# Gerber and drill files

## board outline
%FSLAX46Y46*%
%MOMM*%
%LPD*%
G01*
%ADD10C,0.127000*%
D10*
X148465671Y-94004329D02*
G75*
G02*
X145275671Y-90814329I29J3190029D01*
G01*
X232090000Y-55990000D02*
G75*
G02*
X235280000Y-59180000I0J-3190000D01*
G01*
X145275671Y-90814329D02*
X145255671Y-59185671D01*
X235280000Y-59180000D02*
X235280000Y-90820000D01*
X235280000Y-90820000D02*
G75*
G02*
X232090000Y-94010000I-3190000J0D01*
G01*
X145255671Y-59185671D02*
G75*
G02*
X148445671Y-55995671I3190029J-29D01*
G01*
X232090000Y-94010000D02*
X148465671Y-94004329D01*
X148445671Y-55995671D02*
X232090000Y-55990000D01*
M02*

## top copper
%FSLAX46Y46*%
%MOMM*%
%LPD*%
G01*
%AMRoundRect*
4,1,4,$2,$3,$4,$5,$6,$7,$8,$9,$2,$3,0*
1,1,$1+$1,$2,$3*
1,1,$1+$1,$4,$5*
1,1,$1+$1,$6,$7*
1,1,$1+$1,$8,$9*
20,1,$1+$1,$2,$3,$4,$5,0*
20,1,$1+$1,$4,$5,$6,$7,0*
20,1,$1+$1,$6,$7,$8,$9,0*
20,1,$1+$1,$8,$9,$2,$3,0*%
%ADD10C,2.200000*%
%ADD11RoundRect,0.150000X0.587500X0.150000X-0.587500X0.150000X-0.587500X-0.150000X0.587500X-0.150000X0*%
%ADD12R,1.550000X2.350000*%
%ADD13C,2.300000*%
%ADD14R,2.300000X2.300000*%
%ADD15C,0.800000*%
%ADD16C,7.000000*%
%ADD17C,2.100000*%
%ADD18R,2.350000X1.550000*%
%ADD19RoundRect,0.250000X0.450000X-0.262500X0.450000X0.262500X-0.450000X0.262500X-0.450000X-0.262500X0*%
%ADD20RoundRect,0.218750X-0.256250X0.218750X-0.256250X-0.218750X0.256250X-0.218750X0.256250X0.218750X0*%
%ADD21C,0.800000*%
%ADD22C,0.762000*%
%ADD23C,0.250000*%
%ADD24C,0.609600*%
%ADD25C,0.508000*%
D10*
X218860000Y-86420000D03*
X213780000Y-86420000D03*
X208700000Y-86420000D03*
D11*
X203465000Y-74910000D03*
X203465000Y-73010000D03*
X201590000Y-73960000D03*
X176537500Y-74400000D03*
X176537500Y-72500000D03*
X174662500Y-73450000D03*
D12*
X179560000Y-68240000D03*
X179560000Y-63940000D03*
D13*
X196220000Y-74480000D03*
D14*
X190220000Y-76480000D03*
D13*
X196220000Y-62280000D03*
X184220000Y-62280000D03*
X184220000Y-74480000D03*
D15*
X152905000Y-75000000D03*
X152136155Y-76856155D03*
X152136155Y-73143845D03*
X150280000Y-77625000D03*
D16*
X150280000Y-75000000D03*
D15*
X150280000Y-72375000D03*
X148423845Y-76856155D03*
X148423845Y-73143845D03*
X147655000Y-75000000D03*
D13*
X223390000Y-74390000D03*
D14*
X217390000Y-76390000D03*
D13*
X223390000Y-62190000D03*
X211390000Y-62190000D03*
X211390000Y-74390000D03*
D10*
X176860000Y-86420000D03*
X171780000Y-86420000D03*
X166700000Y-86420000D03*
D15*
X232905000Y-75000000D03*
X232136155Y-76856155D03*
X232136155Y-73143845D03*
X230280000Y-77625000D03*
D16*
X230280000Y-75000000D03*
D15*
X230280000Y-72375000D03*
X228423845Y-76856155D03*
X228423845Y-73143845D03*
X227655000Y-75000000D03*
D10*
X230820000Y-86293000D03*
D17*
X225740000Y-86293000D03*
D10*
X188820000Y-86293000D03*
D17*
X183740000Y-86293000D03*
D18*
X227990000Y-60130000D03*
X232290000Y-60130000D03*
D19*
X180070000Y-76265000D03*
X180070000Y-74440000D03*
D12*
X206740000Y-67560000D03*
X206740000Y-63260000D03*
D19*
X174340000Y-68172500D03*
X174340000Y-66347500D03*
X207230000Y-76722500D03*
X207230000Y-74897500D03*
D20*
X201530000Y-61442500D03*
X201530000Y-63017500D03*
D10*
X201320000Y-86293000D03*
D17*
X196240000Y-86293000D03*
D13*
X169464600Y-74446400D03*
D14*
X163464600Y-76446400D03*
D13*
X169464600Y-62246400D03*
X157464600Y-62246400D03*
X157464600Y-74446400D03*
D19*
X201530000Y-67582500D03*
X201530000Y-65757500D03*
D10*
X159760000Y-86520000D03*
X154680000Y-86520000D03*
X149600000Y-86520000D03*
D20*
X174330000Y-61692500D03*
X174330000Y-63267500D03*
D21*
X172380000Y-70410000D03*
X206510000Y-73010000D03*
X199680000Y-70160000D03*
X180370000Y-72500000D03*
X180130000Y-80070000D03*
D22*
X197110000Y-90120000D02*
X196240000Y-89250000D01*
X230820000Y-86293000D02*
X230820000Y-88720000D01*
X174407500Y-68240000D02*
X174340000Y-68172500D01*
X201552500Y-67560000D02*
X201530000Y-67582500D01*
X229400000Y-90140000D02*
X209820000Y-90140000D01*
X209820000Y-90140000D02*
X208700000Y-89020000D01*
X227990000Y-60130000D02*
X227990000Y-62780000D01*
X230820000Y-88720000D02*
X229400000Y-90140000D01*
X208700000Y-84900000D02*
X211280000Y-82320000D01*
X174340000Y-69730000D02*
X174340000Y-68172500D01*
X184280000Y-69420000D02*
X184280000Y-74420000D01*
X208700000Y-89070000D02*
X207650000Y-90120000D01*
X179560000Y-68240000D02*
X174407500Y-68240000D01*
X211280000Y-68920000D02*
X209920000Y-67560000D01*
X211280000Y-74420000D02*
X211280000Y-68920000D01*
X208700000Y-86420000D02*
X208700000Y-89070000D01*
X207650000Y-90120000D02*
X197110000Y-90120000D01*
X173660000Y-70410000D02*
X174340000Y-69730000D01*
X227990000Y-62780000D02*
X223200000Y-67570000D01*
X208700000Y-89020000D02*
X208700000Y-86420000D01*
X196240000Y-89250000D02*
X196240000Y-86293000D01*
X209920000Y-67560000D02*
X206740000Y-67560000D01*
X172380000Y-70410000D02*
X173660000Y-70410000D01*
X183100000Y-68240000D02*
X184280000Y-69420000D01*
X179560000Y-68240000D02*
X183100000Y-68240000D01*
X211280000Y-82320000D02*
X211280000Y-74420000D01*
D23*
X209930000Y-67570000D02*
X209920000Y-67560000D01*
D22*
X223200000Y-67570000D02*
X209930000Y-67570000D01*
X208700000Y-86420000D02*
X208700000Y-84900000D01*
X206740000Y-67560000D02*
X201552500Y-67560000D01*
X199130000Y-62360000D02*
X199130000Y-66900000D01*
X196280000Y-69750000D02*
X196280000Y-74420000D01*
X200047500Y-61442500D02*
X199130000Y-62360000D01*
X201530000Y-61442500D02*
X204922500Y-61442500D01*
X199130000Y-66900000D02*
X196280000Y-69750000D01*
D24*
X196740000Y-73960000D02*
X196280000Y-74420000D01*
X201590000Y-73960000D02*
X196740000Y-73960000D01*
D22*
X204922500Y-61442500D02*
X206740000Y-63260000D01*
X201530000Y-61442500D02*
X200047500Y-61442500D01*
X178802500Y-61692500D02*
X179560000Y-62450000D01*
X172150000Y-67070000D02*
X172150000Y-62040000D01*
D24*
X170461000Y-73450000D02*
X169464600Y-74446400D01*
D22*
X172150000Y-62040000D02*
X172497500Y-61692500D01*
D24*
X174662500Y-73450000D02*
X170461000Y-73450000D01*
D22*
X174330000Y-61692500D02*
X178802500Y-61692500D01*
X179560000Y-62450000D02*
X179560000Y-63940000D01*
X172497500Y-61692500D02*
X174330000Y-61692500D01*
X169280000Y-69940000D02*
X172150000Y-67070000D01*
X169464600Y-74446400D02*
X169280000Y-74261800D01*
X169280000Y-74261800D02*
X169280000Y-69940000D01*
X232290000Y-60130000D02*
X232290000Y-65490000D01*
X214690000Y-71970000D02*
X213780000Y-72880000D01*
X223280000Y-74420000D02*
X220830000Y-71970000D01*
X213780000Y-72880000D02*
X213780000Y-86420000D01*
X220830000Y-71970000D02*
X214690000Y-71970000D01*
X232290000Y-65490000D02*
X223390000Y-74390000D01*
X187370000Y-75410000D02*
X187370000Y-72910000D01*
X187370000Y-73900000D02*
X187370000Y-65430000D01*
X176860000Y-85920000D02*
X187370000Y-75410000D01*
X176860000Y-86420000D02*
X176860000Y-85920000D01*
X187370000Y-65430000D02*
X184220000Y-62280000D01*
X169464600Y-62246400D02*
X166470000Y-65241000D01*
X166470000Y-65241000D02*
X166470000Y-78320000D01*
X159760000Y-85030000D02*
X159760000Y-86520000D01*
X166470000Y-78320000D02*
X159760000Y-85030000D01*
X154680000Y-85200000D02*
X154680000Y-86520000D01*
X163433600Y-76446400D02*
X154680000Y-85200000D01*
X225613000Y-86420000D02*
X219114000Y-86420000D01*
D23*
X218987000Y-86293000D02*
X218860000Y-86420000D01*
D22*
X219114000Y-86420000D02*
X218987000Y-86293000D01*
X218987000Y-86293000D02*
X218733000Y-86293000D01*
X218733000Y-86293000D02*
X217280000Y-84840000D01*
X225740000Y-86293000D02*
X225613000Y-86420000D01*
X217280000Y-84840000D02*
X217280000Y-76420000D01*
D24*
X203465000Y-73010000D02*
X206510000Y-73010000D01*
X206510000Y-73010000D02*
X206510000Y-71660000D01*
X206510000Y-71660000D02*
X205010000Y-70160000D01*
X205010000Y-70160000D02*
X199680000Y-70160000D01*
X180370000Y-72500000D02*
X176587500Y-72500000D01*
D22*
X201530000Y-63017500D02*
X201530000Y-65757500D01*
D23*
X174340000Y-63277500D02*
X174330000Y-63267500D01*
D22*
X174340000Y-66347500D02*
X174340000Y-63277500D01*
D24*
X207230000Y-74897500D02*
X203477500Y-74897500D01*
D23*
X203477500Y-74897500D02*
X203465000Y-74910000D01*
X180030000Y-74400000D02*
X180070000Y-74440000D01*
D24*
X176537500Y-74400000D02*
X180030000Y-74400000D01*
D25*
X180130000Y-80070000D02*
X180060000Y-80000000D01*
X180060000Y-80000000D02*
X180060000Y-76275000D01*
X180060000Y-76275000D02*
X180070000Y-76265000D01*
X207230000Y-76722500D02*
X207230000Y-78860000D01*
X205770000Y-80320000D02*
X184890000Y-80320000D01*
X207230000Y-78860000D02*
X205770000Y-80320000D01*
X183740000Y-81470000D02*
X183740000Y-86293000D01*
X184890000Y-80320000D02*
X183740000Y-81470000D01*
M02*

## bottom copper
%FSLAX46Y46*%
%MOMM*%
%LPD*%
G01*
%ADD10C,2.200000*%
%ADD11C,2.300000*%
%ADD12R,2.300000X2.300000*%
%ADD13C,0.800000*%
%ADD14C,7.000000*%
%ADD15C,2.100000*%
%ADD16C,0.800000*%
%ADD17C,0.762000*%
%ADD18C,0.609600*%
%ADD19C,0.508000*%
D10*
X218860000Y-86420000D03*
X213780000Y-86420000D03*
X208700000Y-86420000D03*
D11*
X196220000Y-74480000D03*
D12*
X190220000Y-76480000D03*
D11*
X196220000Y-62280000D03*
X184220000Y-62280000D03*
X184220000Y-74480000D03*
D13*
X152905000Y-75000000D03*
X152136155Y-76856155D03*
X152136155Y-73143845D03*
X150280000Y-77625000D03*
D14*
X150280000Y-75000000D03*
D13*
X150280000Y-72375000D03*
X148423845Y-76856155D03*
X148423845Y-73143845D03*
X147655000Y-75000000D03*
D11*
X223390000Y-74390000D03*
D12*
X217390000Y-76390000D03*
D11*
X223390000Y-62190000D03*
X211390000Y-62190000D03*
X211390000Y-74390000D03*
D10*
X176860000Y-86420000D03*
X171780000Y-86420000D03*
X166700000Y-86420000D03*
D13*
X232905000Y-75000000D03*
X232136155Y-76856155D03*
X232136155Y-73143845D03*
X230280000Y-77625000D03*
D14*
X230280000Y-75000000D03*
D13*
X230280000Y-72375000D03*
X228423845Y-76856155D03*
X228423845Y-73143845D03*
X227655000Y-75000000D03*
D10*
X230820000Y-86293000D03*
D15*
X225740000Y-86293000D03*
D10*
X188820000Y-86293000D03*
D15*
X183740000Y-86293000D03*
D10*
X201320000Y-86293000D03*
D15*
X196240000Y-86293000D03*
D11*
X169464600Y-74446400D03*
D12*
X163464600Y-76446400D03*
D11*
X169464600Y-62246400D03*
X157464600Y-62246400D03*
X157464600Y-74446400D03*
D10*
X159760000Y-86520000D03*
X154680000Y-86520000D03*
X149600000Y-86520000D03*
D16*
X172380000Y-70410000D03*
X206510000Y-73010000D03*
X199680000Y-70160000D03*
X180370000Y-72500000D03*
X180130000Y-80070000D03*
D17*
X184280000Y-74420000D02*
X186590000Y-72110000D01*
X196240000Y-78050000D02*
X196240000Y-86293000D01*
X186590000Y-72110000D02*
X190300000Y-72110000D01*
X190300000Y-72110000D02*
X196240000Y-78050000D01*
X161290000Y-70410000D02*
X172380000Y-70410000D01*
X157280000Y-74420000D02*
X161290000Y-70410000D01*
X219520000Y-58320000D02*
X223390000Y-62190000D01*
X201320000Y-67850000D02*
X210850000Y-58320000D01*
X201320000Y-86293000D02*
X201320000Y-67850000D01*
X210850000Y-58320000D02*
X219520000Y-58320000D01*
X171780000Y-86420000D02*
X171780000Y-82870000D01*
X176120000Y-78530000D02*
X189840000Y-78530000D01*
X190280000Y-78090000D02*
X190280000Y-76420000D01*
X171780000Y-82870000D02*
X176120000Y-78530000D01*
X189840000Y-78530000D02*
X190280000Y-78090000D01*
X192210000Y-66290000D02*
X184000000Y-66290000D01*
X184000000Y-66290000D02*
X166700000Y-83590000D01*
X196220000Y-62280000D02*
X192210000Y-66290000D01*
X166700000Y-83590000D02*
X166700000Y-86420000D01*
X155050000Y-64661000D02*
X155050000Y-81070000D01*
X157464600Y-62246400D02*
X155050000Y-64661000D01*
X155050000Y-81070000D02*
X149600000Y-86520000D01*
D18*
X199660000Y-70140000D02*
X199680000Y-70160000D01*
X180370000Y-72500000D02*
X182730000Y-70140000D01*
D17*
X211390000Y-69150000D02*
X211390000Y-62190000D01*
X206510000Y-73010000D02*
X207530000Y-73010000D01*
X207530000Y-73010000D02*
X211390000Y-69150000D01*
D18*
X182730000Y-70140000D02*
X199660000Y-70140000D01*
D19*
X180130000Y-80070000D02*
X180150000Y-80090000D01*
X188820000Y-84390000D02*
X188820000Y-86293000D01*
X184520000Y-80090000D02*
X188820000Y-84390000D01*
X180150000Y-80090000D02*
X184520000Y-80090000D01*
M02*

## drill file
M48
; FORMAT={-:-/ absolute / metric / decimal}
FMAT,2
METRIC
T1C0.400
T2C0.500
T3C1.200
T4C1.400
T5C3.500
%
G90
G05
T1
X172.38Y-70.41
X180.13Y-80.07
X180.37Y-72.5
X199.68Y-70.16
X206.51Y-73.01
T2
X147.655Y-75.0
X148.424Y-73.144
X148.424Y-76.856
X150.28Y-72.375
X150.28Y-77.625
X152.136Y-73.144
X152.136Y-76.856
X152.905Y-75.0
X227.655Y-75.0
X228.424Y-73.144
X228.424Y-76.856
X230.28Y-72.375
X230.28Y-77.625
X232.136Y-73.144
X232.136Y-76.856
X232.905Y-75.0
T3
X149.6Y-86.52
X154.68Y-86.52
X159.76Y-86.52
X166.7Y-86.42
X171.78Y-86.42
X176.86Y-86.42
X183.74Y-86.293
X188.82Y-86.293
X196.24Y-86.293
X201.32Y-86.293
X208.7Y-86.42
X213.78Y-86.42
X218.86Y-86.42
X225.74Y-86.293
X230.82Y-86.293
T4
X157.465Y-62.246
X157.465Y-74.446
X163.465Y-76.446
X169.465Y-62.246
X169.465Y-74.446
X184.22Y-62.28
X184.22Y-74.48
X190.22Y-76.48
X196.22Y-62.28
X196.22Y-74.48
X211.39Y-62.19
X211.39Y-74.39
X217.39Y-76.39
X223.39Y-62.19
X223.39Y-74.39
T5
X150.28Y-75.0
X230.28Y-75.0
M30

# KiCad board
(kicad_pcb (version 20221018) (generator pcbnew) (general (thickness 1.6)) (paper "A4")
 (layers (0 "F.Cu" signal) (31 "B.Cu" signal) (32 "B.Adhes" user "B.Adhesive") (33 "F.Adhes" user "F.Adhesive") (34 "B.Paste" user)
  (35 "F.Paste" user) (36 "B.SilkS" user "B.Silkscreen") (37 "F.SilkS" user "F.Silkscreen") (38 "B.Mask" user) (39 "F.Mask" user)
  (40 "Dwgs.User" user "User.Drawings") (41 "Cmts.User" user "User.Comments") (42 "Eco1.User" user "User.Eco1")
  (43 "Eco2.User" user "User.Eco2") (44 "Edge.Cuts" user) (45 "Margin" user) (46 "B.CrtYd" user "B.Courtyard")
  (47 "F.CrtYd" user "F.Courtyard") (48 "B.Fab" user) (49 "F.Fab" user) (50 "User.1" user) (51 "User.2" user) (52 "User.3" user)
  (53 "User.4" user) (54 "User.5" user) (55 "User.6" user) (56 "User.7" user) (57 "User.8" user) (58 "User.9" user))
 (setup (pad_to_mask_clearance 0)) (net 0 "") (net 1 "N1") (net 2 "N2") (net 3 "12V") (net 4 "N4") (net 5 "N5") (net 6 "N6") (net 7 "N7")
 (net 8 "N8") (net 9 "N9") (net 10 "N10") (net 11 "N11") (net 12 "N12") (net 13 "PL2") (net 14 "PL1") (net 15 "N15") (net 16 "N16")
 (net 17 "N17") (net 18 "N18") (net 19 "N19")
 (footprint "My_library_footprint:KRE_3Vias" (layer "F.Cu") (at 213.78 86.42 180)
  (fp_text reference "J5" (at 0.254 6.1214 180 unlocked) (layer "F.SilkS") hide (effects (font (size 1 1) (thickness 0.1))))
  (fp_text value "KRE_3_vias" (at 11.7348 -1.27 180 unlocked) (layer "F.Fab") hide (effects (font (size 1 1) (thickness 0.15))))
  (pad "1" thru_hole circle (at -5.08 0 180) (size 2.2 2.2) (drill 1.2) (layers "*.Cu" "*.Mask") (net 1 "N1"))
  (pad "2" thru_hole circle (at 0 0 180) (size 2.2 2.2) (drill 1.2) (layers "*.Cu" "*.Mask") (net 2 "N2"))
  (pad "3" thru_hole circle (at 5.08 0 180) (size 2.2 2.2) (drill 1.2) (layers "*.Cu" "*.Mask") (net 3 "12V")))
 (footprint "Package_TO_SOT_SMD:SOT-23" (layer "F.Cu") (at 202.5275 73.96 180)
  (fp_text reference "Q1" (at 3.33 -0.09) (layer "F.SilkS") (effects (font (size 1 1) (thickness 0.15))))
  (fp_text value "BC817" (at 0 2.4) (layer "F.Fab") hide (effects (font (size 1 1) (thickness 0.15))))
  (pad "1" smd roundrect (at -0.9375 -0.95 180) (size 1.475 0.6) (layers "F.Cu" "F.Paste" "F.Mask") (roundrect_rratio 0.25) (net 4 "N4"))
  (pad "2" smd roundrect (at -0.9375 0.95 180) (size 1.475 0.6) (layers "F.Cu" "F.Paste" "F.Mask") (roundrect_rratio 0.25) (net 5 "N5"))
  (pad "3" smd roundrect (at 0.9375 0 180) (size 1.475 0.6) (layers "F.Cu" "F.Paste" "F.Mask") (roundrect_rratio 0.25) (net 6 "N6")))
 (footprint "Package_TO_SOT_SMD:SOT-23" (layer "F.Cu") (at 175.6 73.45 180)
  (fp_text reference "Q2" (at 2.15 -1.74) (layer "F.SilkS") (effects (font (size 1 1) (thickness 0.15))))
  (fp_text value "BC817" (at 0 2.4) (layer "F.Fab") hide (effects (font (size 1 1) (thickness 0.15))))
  (pad "1" smd roundrect (at -0.9375 -0.95 180) (size 1.475 0.6) (layers "F.Cu" "F.Paste" "F.Mask") (roundrect_rratio 0.25) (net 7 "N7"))
  (pad "2" smd roundrect (at -0.9375 0.95 180) (size 1.475 0.6) (layers "F.Cu" "F.Paste" "F.Mask") (roundrect_rratio 0.25) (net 5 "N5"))
  (pad "3" smd roundrect (at 0.9375 0 180) (size 1.475 0.6) (layers "F.Cu" "F.Paste" "F.Mask") (roundrect_rratio 0.25) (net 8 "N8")))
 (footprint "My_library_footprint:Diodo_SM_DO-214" (layer "F.Cu") (at 179.56 66.09 90)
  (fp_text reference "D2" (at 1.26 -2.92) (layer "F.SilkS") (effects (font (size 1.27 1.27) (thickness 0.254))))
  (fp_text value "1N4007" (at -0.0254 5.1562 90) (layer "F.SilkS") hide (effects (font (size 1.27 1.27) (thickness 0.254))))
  (pad "1" smd rect (at -2.15 0 180) (size 1.55 2.35) (layers "F.Cu" "F.Paste" "F.Mask") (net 3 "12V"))
  (pad "2" smd rect (at 2.15 0 180) (size 1.55 2.35) (layers "F.Cu" "F.Paste" "F.Mask") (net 8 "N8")))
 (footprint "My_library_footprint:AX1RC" (layer "F.Cu") (at 190.22 76.48 90)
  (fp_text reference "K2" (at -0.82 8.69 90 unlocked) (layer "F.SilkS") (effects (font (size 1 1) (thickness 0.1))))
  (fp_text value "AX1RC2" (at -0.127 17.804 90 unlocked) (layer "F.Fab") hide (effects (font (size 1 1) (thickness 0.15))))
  (pad "1" thru_hole circle (at 2 6 90) (size 2.3 2.3) (drill 1.4) (layers "*.Cu" "*.Mask") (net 6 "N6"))
  (pad "2" thru_hole rect (at 0 0 90) (size 2.3 2.3) (drill 1.4) (layers "*.Cu" "*.Mask") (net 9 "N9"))
  (pad "3" thru_hole circle (at 14.2 6 90) (size 2.3 2.3) (drill 1.4) (layers "*.Cu" "*.Mask") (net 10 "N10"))
  (pad "4" thru_hole circle (at 14.2 -6 90) (size 2.3 2.3) (drill 1.4) (layers "*.Cu" "*.Mask") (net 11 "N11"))
  (pad "5" thru_hole circle (at 2 -6 90) (size 2.3 2.3) (drill 1.4) (layers "*.Cu" "*.Mask") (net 3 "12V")))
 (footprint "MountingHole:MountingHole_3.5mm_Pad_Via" (layer "F.Cu") (at 150.28 75 180)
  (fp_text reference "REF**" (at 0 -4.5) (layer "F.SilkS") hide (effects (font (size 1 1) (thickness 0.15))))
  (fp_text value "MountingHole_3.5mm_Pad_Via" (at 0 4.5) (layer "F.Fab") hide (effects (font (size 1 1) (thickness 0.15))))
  (pad "1" thru_hole circle (at -2.625 0 180) (size 0.8 0.8) (drill 0.5) (layers "*.Cu" "*.Mask"))
  (pad "1" thru_hole circle (at -1.856155 -1.856155 180) (size 0.8 0.8) (drill 0.5) (layers "*.Cu" "*.Mask"))
  (pad "1" thru_hole circle (at -1.856155 1.856155 180) (size 0.8 0.8) (drill 0.5) (layers "*.Cu" "*.Mask"))
  (pad "1" thru_hole circle (at 0 -2.625 180) (size 0.8 0.8) (drill 0.5) (layers "*.Cu" "*.Mask"))
  (pad "1" thru_hole circle (at 0 0 180) (size 7 7) (drill 3.5) (layers "*.Cu" "*.Mask"))
  (pad "1" thru_hole circle (at 0 2.625 180) (size 0.8 0.8) (drill 0.5) (layers "*.Cu" "*.Mask"))
  (pad "1" thru_hole circle (at 1.856155 -1.856155 180) (size 0.8 0.8) (drill 0.5) (layers "*.Cu" "*.Mask"))
  (pad "1" thru_hole circle (at 1.856155 1.856155 180) (size 0.8 0.8) (drill 0.5) (layers "*.Cu" "*.Mask"))
  (pad "1" thru_hole circle (at 2.625 0 180) (size 0.8 0.8) (drill 0.5) (layers "*.Cu" "*.Mask")))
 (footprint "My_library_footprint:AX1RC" (layer "F.Cu") (at 217.39 76.39 90)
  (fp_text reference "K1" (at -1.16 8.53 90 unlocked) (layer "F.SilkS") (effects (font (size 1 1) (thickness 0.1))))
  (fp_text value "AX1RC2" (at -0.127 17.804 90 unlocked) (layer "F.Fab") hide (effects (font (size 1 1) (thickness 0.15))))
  (pad "1" thru_hole circle (at 2 6 90) (size 2.3 2.3) (drill 1.4) (layers "*.Cu" "*.Mask") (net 2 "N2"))
  (pad "2" thru_hole rect (at 0 0 90) (size 2.3 2.3) (drill 1.4) (layers "*.Cu" "*.Mask") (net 1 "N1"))
  (pad "3" thru_hole circle (at 14.2 6 90) (size 2.3 2.3) (drill 1.4) (layers "*.Cu" "*.Mask") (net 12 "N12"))
  (pad "4" thru_hole circle (at 14.2 -6 90) (size 2.3 2.3) (drill 1.4) (layers "*.Cu" "*.Mask") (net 5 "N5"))
  (pad "5" thru_hole circle (at 2 -6 90) (size 2.3 2.3) (drill 1.4) (layers "*.Cu" "*.Mask") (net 3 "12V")))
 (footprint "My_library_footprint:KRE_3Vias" (layer "F.Cu") (at 171.78 86.42 180)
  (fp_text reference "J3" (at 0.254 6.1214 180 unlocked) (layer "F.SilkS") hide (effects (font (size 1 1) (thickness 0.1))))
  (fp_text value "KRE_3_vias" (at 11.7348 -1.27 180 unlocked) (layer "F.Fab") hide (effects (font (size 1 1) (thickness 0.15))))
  (pad "1" thru_hole circle (at -5.08 0 180) (size 2.2 2.2) (drill 1.2) (layers "*.Cu" "*.Mask") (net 11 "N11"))
  (pad "2" thru_hole circle (at 0 0 180) (size 2.2 2.2) (drill 1.2) (layers "*.Cu" "*.Mask") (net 9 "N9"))
  (pad "3" thru_hole circle (at 5.08 0 180) (size 2.2 2.2) (drill 1.2) (layers "*.Cu" "*.Mask") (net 10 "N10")))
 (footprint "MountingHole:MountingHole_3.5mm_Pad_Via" (layer "F.Cu") (at 230.28 75 180)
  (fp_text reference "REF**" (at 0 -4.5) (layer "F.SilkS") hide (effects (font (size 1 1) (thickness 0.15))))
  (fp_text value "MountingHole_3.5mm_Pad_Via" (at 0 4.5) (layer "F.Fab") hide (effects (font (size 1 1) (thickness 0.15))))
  (pad "1" thru_hole circle (at -2.625 0 180) (size 0.8 0.8) (drill 0.5) (layers "*.Cu" "*.Mask"))
  (pad "1" thru_hole circle (at -1.856155 -1.856155 180) (size 0.8 0.8) (drill 0.5) (layers "*.Cu" "*.Mask"))
  (pad "1" thru_hole circle (at -1.856155 1.856155 180) (size 0.8 0.8) (drill 0.5) (layers "*.Cu" "*.Mask"))
  (pad "1" thru_hole circle (at 0 -2.625 180) (size 0.8 0.8) (drill 0.5) (layers "*.Cu" "*.Mask"))
  (pad "1" thru_hole circle (at 0 0 180) (size 7 7) (drill 3.5) (layers "*.Cu" "*.Mask"))
  (pad "1" thru_hole circle (at 0 2.625 180) (size 0.8 0.8) (drill 0.5) (layers "*.Cu" "*.Mask"))
  (pad "1" thru_hole circle (at 1.856155 -1.856155 180) (size 0.8 0.8) (drill 0.5) (layers "*.Cu" "*.Mask"))
  (pad "1" thru_hole circle (at 1.856155 1.856155 180) (size 0.8 0.8) (drill 0.5) (layers "*.Cu" "*.Mask"))
  (pad "1" thru_hole circle (at 2.625 0 180) (size 0.8 0.8) (drill 0.5) (layers "*.Cu" "*.Mask")))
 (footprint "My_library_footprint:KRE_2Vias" (layer "F.Cu") (at 228.28 86.42 180)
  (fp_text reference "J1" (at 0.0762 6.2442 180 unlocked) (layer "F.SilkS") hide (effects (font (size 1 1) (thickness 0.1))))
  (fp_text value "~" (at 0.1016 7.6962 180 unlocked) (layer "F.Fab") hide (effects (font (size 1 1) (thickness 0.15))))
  (pad "1" thru_hole circle (at -2.54 0.127 180) (size 2.2 2.2) (drill 1.2) (layers "*.Cu" "*.Mask") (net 3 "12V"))
  (pad "2" thru_hole circle (at 2.54 0.127 180) (size 2.1 2.1) (drill 1.2) (layers "*.Cu" "*.Mask") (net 1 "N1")))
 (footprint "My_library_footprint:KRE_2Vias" (layer "F.Cu") (at 186.28 86.42 180)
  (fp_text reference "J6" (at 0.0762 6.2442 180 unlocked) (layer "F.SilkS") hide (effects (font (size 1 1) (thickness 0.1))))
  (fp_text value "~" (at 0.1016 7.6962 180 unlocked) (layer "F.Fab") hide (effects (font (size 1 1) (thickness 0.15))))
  (pad "1" thru_hole circle (at -2.54 0.127 180) (size 2.2 2.2) (drill 1.2) (layers "*.Cu" "*.Mask") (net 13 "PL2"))
  (pad "2" thru_hole circle (at 2.54 0.127 180) (size 2.1 2.1) (drill 1.2) (layers "*.Cu" "*.Mask") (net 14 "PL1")))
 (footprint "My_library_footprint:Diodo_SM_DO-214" (layer "F.Cu") (at 230.14 60.13)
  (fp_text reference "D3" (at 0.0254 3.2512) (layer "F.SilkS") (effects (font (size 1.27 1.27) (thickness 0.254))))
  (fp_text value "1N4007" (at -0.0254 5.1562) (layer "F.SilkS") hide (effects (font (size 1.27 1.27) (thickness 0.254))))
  (pad "1" smd rect (at -2.15 0 90) (size 1.55 2.35) (layers "F.Cu" "F.Paste" "F.Mask") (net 3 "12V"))
  (pad "2" smd rect (at 2.15 0 90) (size 1.55 2.35) (layers "F.Cu" "F.Paste" "F.Mask") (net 2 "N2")))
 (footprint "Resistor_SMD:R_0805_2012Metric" (layer "F.Cu") (at 180.07 75.3525 90)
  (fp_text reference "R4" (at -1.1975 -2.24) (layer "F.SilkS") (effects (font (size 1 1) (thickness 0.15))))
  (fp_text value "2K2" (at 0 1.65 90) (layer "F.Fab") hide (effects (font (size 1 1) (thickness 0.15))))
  (pad "1" smd roundrect (at -0.9125 0 90) (size 1.025 1.4) (layers "F.Cu" "F.Paste" "F.Mask") (roundrect_rratio 0.243902439) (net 13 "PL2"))
  (pad "2" smd roundrect (at 0.9125 0 90) (size 1.025 1.4) (layers "F.Cu" "F.Paste" "F.Mask") (roundrect_rratio 0.243902439) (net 7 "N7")))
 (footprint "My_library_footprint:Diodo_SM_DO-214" (layer "F.Cu") (at 206.74 65.41 90)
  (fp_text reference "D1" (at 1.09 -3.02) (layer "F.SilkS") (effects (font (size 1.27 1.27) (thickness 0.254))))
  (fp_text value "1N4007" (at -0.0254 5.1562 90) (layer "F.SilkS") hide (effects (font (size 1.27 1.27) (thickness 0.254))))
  (pad "1" smd rect (at -2.15 0 180) (size 1.55 2.35) (layers "F.Cu" "F.Paste" "F.Mask") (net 3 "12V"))
  (pad "2" smd rect (at 2.15 0 180) (size 1.55 2.35) (layers "F.Cu" "F.Paste" "F.Mask") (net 6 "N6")))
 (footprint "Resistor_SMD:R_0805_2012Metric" (layer "F.Cu") (at 174.34 67.26 90)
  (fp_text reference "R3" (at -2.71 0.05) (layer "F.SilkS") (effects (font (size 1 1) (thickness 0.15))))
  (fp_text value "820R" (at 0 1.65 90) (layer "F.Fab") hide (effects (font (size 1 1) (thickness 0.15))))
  (pad "1" smd roundrect (at -0.9125 0 90) (size 1.025 1.4) (layers "F.Cu" "F.Paste" "F.Mask") (roundrect_rratio 0.243902439) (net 3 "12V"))
  (pad "2" smd roundrect (at 0.9125 0 90) (size 1.025 1.4) (layers "F.Cu" "F.Paste" "F.Mask") (roundrect_rratio 0.243902439) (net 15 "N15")))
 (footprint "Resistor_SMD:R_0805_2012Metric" (layer "F.Cu") (at 207.23 75.81 90)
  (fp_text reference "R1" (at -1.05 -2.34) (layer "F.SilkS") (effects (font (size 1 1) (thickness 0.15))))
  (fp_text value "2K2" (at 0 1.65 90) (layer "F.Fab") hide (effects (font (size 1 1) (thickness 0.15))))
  (pad "1" smd roundrect (at -0.9125 0 90) (size 1.025 1.4) (layers "F.Cu" "F.Paste" "F.Mask") (roundrect_rratio 0.243902439) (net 14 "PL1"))
  (pad "2" smd roundrect (at 0.9125 0 90) (size 1.025 1.4) (layers "F.Cu" "F.Paste" "F.Mask") (roundrect_rratio 0.243902439) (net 4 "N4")))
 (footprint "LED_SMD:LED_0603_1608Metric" (layer "F.Cu") (at 201.53 62.23 -90)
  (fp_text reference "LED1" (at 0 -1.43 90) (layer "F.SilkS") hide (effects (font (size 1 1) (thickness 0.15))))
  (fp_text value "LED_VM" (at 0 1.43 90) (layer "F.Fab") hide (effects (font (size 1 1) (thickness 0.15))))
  (pad "1" smd roundrect (at -0.7875 0 270) (size 0.875 0.95) (layers "F.Cu" "F.Paste" "F.Mask") (roundrect_rratio 0.25) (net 6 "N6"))
  (pad "2" smd roundrect (at 0.7875 0 270) (size 0.875 0.95) (layers "F.Cu" "F.Paste" "F.Mask") (roundrect_rratio 0.25) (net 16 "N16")))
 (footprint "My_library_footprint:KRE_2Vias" (layer "F.Cu") (at 198.78 86.42 180)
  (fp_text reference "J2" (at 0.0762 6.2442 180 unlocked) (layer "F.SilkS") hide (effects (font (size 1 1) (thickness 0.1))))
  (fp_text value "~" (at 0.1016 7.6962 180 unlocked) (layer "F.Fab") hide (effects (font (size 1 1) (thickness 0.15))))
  (pad "1" thru_hole circle (at -2.54 0.127 180) (size 2.2 2.2) (drill 1.2) (layers "*.Cu" "*.Mask") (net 12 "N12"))
  (pad "2" thru_hole circle (at 2.54 0.127 180) (size 2.1 2.1) (drill 1.2) (layers "*.Cu" "*.Mask") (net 3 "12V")))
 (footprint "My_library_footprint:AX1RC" (layer "F.Cu") (at 163.4646 76.4464 90)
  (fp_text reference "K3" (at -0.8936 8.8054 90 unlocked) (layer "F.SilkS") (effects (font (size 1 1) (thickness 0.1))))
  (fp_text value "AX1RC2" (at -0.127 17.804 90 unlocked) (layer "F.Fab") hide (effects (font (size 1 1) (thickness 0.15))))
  (pad "1" thru_hole circle (at 2 6 90) (size 2.3 2.3) (drill 1.4) (layers "*.Cu" "*.Mask") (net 8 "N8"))
  (pad "2" thru_hole rect (at 0 0 90) (size 2.3 2.3) (drill 1.4) (layers "*.Cu" "*.Mask") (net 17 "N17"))
  (pad "3" thru_hole circle (at 14.2 6 90) (size 2.3 2.3) (drill 1.4) (layers "*.Cu" "*.Mask") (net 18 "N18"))
  (pad "4" thru_hole circle (at 14.2 -6 90) (size 2.3 2.3) (drill 1.4) (layers "*.Cu" "*.Mask") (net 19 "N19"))
  (pad "5" thru_hole circle (at 2 -6 90) (size 2.3 2.3) (drill 1.4) (layers "*.Cu" "*.Mask") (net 3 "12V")))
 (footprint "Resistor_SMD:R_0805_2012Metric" (layer "F.Cu") (at 201.53 66.67 90)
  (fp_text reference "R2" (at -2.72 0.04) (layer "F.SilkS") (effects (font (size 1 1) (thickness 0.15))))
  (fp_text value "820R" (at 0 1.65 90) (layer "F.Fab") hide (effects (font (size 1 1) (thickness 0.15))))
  (pad "1" smd roundrect (at -0.9125 0 90) (size 1.025 1.4) (layers "F.Cu" "F.Paste" "F.Mask") (roundrect_rratio 0.243902439) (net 3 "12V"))
  (pad "2" smd roundrect (at 0.9125 0 90) (size 1.025 1.4) (layers "F.Cu" "F.Paste" "F.Mask") (roundrect_rratio 0.243902439) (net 16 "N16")))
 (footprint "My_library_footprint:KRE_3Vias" (layer "F.Cu") (at 154.68 86.52 180)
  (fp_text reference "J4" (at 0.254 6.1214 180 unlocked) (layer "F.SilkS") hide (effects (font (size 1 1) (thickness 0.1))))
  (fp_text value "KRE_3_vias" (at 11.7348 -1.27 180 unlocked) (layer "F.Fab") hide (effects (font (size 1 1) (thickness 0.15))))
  (pad "1" thru_hole circle (at -5.08 0 180) (size 2.2 2.2) (drill 1.2) (layers "*.Cu" "*.Mask") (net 18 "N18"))
  (pad "2" thru_hole circle (at 0 0 180) (size 2.2 2.2) (drill 1.2) (layers "*.Cu" "*.Mask") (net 17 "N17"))
  (pad "3" thru_hole circle (at 5.08 0 180) (size 2.2 2.2) (drill 1.2) (layers "*.Cu" "*.Mask") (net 19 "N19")))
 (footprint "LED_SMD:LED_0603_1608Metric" (layer "F.Cu") (at 174.33 62.48 -90)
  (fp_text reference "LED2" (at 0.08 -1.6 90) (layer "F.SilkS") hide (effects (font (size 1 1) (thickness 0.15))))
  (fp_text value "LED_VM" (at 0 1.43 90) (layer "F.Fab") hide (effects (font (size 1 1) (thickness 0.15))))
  (pad "1" smd roundrect (at -0.7875 0 270) (size 0.875 0.95) (layers "F.Cu" "F.Paste" "F.Mask") (roundrect_rratio 0.25) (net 8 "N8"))
  (pad "2" smd roundrect (at 0.7875 0 270) (size 0.875 0.95) (layers "F.Cu" "F.Paste" "F.Mask") (roundrect_rratio 0.25) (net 15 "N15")))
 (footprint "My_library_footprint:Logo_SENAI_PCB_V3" (layer "B.Cu") (at 225.837083 67.344083 180)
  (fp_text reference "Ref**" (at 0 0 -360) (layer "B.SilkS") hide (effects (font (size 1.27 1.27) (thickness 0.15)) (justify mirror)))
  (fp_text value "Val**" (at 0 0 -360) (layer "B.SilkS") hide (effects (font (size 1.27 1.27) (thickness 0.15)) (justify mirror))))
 (gr_arc (start 148.465671 94.004329) (mid 146.21 93.07) (end 145.275671 90.814329) (stroke (width 0.127) (type default))
  (layer "Edge.Cuts"))
 (gr_arc (start 232.09 55.99) (mid 234.345671 56.924329) (end 235.28 59.18) (stroke (width 0.127) (type default)) (layer "Edge.Cuts"))
 (gr_line (start 145.275671 90.814329) (end 145.255671 59.185671) (stroke (width 0.127) (type default)) (layer "Edge.Cuts"))
 (gr_line (start 235.28 59.18) (end 235.28 90.82) (stroke (width 0.127) (type default)) (layer "Edge.Cuts"))
 (gr_arc (start 235.28 90.82) (mid 234.345671 93.075671) (end 232.09 94.01) (stroke (width 0.127) (type default)) (layer "Edge.Cuts"))
 (gr_arc (start 145.255671 59.185671) (mid 146.19 56.93) (end 148.445671 55.995671) (stroke (width 0.127) (type default))
  (layer "Edge.Cuts"))
 (gr_line (start 232.09 94.01) (end 148.465671 94.004329) (stroke (width 0.127) (type default)) (layer "Edge.Cuts"))
 (gr_line (start 148.445671 55.995671) (end 232.09 55.99) (stroke (width 0.127) (type default)) (layer "Edge.Cuts"))
 (segment (start 197.11 90.12) (end 196.24 89.25) (width 0.762) (layer "F.Cu") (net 3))
 (segment (start 230.82 86.293) (end 230.82 88.72) (width 0.762) (layer "F.Cu") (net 3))
 (segment (start 174.4075 68.24) (end 174.34 68.1725) (width 0.762) (layer "F.Cu") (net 3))
 (segment (start 201.5525 67.56) (end 201.53 67.5825) (width 0.762) (layer "F.Cu") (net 3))
 (segment (start 229.4 90.14) (end 209.82 90.14) (width 0.762) (layer "F.Cu") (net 3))
 (segment (start 209.82 90.14) (end 208.7 89.02) (width 0.762) (layer "F.Cu") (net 3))
 (segment (start 227.99 60.13) (end 227.99 62.78) (width 0.762) (layer "F.Cu") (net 3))
 (segment (start 230.82 88.72) (end 229.4 90.14) (width 0.762) (layer "F.Cu") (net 3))
 (segment (start 208.7 84.9) (end 211.28 82.32) (width 0.762) (layer "F.Cu") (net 3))
 (segment (start 174.34 69.73) (end 174.34 68.1725) (width 0.762) (layer "F.Cu") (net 3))
 (segment (start 184.28 69.42) (end 184.28 74.42) (width 0.762) (layer "F.Cu") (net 3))
 (segment (start 208.7 89.07) (end 207.65 90.12) (width 0.762) (layer "F.Cu") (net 3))
 (segment (start 179.56 68.24) (end 174.4075 68.24) (width 0.762) (layer "F.Cu") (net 3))
 (segment (start 211.28 68.92) (end 209.92 67.56) (width 0.762) (layer "F.Cu") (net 3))
 (segment (start 211.28 74.42) (end 211.28 68.92) (width 0.762) (layer "F.Cu") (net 3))
 (segment (start 208.7 86.42) (end 208.7 89.07) (width 0.762) (layer "F.Cu") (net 3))
 (segment (start 207.65 90.12) (end 197.11 90.12) (width 0.762) (layer "F.Cu") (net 3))
 (segment (start 173.66 70.41) (end 174.34 69.73) (width 0.762) (layer "F.Cu") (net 3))
 (segment (start 227.99 62.78) (end 223.2 67.57) (width 0.762) (layer "F.Cu") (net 3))
 (segment (start 208.7 89.02) (end 208.7 86.42) (width 0.762) (layer "F.Cu") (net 3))
 (segment (start 196.24 89.25) (end 196.24 86.293) (width 0.762) (layer "F.Cu") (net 3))
 (segment (start 209.92 67.56) (end 206.74 67.56) (width 0.762) (layer "F.Cu") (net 3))
 (segment (start 172.38 70.41) (end 173.66 70.41) (width 0.762) (layer "F.Cu") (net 3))
 (segment (start 183.1 68.24) (end 184.28 69.42) (width 0.762) (layer "F.Cu") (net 3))
 (segment (start 179.56 68.24) (end 183.1 68.24) (width 0.762) (layer "F.Cu") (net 3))
 (segment (start 211.28 82.32) (end 211.28 74.42) (width 0.762) (layer "F.Cu") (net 3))
 (segment (start 209.93 67.57) (end 209.92 67.56) (width 0.25) (layer "F.Cu") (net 3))
 (segment (start 223.2 67.57) (end 209.93 67.57) (width 0.762) (layer "F.Cu") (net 3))
 (segment (start 208.7 86.42) (end 208.7 84.9) (width 0.762) (layer "F.Cu") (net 3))
 (segment (start 206.74 67.56) (end 201.5525 67.56) (width 0.762) (layer "F.Cu") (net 3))
 (via (at 172.38 70.41) (size 0.8) (drill 0.4) (layers "F.Cu" "B.Cu") (free) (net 3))
 (segment (start 184.28 74.42) (end 186.59 72.11) (width 0.762) (layer "B.Cu") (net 3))
 (segment (start 196.24 78.05) (end 196.24 86.293) (width 0.762) (layer "B.Cu") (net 3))
 (segment (start 186.59 72.11) (end 190.3 72.11) (width 0.762) (layer "B.Cu") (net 3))
 (segment (start 190.3 72.11) (end 196.24 78.05) (width 0.762) (layer "B.Cu") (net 3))
 (segment (start 161.29 70.41) (end 172.38 70.41) (width 0.762) (layer "B.Cu") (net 3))
 (segment (start 157.28 74.42) (end 161.29 70.41) (width 0.762) (layer "B.Cu") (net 3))
 (segment (start 199.13 62.36) (end 199.13 66.9) (width 0.762) (layer "F.Cu") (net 6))
 (segment (start 196.28 69.75) (end 196.28 74.42) (width 0.762) (layer "F.Cu") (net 6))
 (segment (start 200.0475 61.4425) (end 199.13 62.36) (width 0.762) (layer "F.Cu") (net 6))
 (segment (start 201.53 61.4425) (end 204.9225 61.4425) (width 0.762) (layer "F.Cu") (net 6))
 (segment (start 199.13 66.9) (end 196.28 69.75) (width 0.762) (layer "F.Cu") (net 6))
 (segment (start 196.74 73.96) (end 196.28 74.42) (width 0.6096) (layer "F.Cu") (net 6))
 (segment (start 201.59 73.96) (end 196.74 73.96) (width 0.6096) (layer "F.Cu") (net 6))
 (segment (start 204.9225 61.4425) (end 206.74 63.26) (width 0.762) (layer "F.Cu") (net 6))
 (segment (start 201.53 61.4425) (end 200.0475 61.4425) (width 0.762) (layer "F.Cu") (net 6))
 (segment (start 178.8025 61.6925) (end 179.56 62.45) (width 0.762) (layer "F.Cu") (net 8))
 (segment (start 172.15 67.07) (end 172.15 62.04) (width 0.762) (layer "F.Cu") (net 8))
 (segment (start 170.461 73.45) (end 169.4646 74.4464) (width 0.6096) (layer "F.Cu") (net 8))
 (segment (start 172.15 62.04) (end 172.4975 61.6925) (width 0.762) (layer "F.Cu") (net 8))
 (segment (start 174.6625 73.45) (end 170.461 73.45) (width 0.6096) (layer "F.Cu") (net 8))
 (segment (start 174.33 61.6925) (end 178.8025 61.6925) (width 0.762) (layer "F.Cu") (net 8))
 (segment (start 179.56 62.45) (end 179.56 63.94) (width 0.762) (layer "F.Cu") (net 8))
 (segment (start 172.4975 61.6925) (end 174.33 61.6925) (width 0.762) (layer "F.Cu") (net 8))
 (segment (start 169.28 69.94) (end 172.15 67.07) (width 0.762) (layer "F.Cu") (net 8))
 (segment (start 169.4646 74.4464) (end 169.28 74.2618) (width 0.762) (layer "F.Cu") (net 8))
 (segment (start 169.28 74.2618) (end 169.28 69.94) (width 0.762) (layer "F.Cu") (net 8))
 (segment (start 232.29 60.13) (end 232.29 65.49) (width 0.762) (layer "F.Cu") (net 2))
 (segment (start 214.69 71.97) (end 213.78 72.88) (width 0.762) (layer "F.Cu") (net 2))
 (segment (start 223.28 74.42) (end 220.83 71.97) (width 0.762) (layer "F.Cu") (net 2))
 (segment (start 213.78 72.88) (end 213.78 86.42) (width 0.762) (layer "F.Cu") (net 2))
 (segment (start 220.83 71.97) (end 214.69 71.97) (width 0.762) (layer "F.Cu") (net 2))
 (segment (start 232.29 65.49) (end 223.39 74.39) (width 0.762) (layer "F.Cu") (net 2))
 (segment (start 219.52 58.32) (end 223.39 62.19) (width 0.762) (layer "B.Cu") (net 12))
 (segment (start 201.32 67.85) (end 210.85 58.32) (width 0.762) (layer "B.Cu") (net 12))
 (segment (start 201.32 86.293) (end 201.32 67.85) (width 0.762) (layer "B.Cu") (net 12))
 (segment (start 210.85 58.32) (end 219.52 58.32) (width 0.762) (layer "B.Cu") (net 12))
 (segment (start 187.37 75.41) (end 187.37 72.91) (width 0.762) (layer "F.Cu") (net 11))
 (segment (start 187.37 73.9) (end 187.37 65.43) (width 0.762) (layer "F.Cu") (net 11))
 (segment (start 176.86 85.92) (end 187.37 75.41) (width 0.762) (layer "F.Cu") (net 11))
 (segment (start 176.86 86.42) (end 176.86 85.92) (width 0.762) (layer "F.Cu") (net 11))
 (segment (start 187.37 65.43) (end 184.22 62.28) (width 0.762) (layer "F.Cu") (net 11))
 (segment (start 171.78 86.42) (end 171.78 82.87) (width 0.762) (layer "B.Cu") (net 9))
 (segment (start 176.12 78.53) (end 189.84 78.53) (width 0.762) (layer "B.Cu") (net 9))
 (segment (start 190.28 78.09) (end 190.28 76.42) (width 0.762) (layer "B.Cu") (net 9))
 (segment (start 171.78 82.87) (end 176.12 78.53) (width 0.762) (layer "B.Cu") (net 9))
 (segment (start 189.84 78.53) (end 190.28 78.09) (width 0.762) (layer "B.Cu") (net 9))
 (segment (start 192.21 66.29) (end 184 66.29) (width 0.762) (layer "B.Cu") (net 10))
 (segment (start 184 66.29) (end 166.7 83.59) (width 0.762) (layer "B.Cu") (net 10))
 (segment (start 196.22 62.28) (end 192.21 66.29) (width 0.762) (layer "B.Cu") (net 10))
 (segment (start 166.7 83.59) (end 166.7 86.42) (width 0.762) (layer "B.Cu") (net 10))
 (segment (start 169.4646 62.2464) (end 166.47 65.241) (width 0.762) (layer "F.Cu") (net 18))
 (segment (start 166.47 65.241) (end 166.47 78.32) (width 0.762) (layer "F.Cu") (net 18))
 (segment (start 159.76 85.03) (end 159.76 86.52) (width 0.762) (layer "F.Cu") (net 18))
 (segment (start 166.47 78.32) (end 159.76 85.03) (width 0.762) (layer "F.Cu") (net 18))
 (segment (start 154.68 85.2) (end 154.68 86.52) (width 0.762) (layer "F.Cu") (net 17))
 (segment (start 163.4336 76.4464) (end 154.68 85.2) (width 0.762) (layer "F.Cu") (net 17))
 (segment (start 155.05 64.661) (end 155.05 81.07) (width 0.762) (layer "B.Cu") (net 19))
 (segment (start 157.4646 62.2464) (end 155.05 64.661) (width 0.762) (layer "B.Cu") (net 19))
 (segment (start 155.05 81.07) (end 149.6 86.52) (width 0.762) (layer "B.Cu") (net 19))
 (segment (start 225.613 86.42) (end 219.114 86.42) (width 0.762) (layer "F.Cu") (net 1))
 (segment (start 218.987 86.293) (end 218.86 86.42) (width 0.25) (layer "F.Cu") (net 1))
 (segment (start 219.114 86.42) (end 218.987 86.293) (width 0.762) (layer "F.Cu") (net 1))
 (segment (start 218.987 86.293) (end 218.733 86.293) (width 0.762) (layer "F.Cu") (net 1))
 (segment (start 218.733 86.293) (end 217.28 84.84) (width 0.762) (layer "F.Cu") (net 1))
 (segment (start 225.74 86.293) (end 225.613 86.42) (width 0.762) (layer "F.Cu") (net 1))
 (segment (start 217.28 84.84) (end 217.28 76.42) (width 0.762) (layer "F.Cu") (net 1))
 (segment (start 203.465 73.01) (end 206.51 73.01) (width 0.6096) (layer "F.Cu") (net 5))
 (segment (start 206.51 73.01) (end 206.51 71.66) (width 0.6096) (layer "F.Cu") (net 5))
 (segment (start 206.51 71.66) (end 205.01 70.16) (width 0.6096) (layer "F.Cu") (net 5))
 (segment (start 205.01 70.16) (end 199.68 70.16) (width 0.6096) (layer "F.Cu") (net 5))
 (segment (start 180.37 72.5) (end 176.5875 72.5) (width 0.6096) (layer "F.Cu") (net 5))
 (via (at 206.51 73.01) (size 0.8) (drill 0.4) (layers "F.Cu" "B.Cu") (free) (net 5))
 (via (at 199.68 70.16) (size 0.8) (drill 0.4) (layers "F.Cu" "B.Cu") (free) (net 5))
 (via (at 180.37 72.5) (size 0.8) (drill 0.4) (layers "F.Cu" "B.Cu") (free) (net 5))
 (segment (start 199.66 70.14) (end 199.68 70.16) (width 0.6096) (layer "B.Cu") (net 5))
 (segment (start 180.37 72.5) (end 182.73 70.14) (width 0.6096) (layer "B.Cu") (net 5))
 (segment (start 211.39 69.15) (end 211.39 62.19) (width 0.762) (layer "B.Cu") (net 5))
 (segment (start 206.51 73.01) (end 207.53 73.01) (width 0.762) (layer "B.Cu") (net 5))
 (segment (start 207.53 73.01) (end 211.39 69.15) (width 0.762) (layer "B.Cu") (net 5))
 (segment (start 182.73 70.14) (end 199.66 70.14) (width 0.6096) (layer "B.Cu") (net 5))
 (segment (start 201.53 63.0175) (end 201.53 65.7575) (width 0.762) (layer "F.Cu") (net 16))
 (segment (start 174.34 63.2775) (end 174.33 63.2675) (width 0.25) (layer "F.Cu") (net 15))
 (segment (start 174.34 66.3475) (end 174.34 63.2775) (width 0.762) (layer "F.Cu") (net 15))
 (segment (start 207.23 74.8975) (end 203.4775 74.8975) (width 0.6096) (layer "F.Cu") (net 4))
 (segment (start 203.4775 74.8975) (end 203.465 74.91) (width 0.25) (layer "F.Cu") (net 4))
 (segment (start 180.03 74.4) (end 180.07 74.44) (width 0.25) (layer "F.Cu") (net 7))
 (segment (start 176.5375 74.4) (end 180.03 74.4) (width 0.6096) (layer "F.Cu") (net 7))
 (segment (start 180.13 80.07) (end 180.06 80) (width 0.508) (layer "F.Cu") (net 13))
 (segment (start 180.06 80) (end 180.06 76.275) (width 0.508) (layer "F.Cu") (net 13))
 (segment (start 180.06 76.275) (end 180.07 76.265) (width 0.508) (layer "F.Cu") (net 13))
 (via (at 180.13 80.07) (size 0.8) (drill 0.4) (layers "F.Cu" "B.Cu") (free) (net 13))
 (segment (start 180.13 80.07) (end 180.15 80.09) (width 0.508) (layer "B.Cu") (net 13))
 (segment (start 188.82 84.39) (end 188.82 86.293) (width 0.508) (layer "B.Cu") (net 13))
 (segment (start 184.52 80.09) (end 188.82 84.39) (width 0.508) (layer "B.Cu") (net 13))
 (segment (start 180.15 80.09) (end 184.52 80.09) (width 0.508) (layer "B.Cu") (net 13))
 (segment (start 207.23 76.7225) (end 207.23 78.86) (width 0.508) (layer "F.Cu") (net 14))
 (segment (start 205.77 80.32) (end 184.89 80.32) (width 0.508) (layer "F.Cu") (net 14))
 (segment (start 207.23 78.86) (end 205.77 80.32) (width 0.508) (layer "F.Cu") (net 14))
 (segment (start 183.74 81.47) (end 183.74 86.293) (width 0.508) (layer "F.Cu") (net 14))
 (segment (start 184.89 80.32) (end 183.74 81.47) (width 0.508) (layer "F.Cu") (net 14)))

